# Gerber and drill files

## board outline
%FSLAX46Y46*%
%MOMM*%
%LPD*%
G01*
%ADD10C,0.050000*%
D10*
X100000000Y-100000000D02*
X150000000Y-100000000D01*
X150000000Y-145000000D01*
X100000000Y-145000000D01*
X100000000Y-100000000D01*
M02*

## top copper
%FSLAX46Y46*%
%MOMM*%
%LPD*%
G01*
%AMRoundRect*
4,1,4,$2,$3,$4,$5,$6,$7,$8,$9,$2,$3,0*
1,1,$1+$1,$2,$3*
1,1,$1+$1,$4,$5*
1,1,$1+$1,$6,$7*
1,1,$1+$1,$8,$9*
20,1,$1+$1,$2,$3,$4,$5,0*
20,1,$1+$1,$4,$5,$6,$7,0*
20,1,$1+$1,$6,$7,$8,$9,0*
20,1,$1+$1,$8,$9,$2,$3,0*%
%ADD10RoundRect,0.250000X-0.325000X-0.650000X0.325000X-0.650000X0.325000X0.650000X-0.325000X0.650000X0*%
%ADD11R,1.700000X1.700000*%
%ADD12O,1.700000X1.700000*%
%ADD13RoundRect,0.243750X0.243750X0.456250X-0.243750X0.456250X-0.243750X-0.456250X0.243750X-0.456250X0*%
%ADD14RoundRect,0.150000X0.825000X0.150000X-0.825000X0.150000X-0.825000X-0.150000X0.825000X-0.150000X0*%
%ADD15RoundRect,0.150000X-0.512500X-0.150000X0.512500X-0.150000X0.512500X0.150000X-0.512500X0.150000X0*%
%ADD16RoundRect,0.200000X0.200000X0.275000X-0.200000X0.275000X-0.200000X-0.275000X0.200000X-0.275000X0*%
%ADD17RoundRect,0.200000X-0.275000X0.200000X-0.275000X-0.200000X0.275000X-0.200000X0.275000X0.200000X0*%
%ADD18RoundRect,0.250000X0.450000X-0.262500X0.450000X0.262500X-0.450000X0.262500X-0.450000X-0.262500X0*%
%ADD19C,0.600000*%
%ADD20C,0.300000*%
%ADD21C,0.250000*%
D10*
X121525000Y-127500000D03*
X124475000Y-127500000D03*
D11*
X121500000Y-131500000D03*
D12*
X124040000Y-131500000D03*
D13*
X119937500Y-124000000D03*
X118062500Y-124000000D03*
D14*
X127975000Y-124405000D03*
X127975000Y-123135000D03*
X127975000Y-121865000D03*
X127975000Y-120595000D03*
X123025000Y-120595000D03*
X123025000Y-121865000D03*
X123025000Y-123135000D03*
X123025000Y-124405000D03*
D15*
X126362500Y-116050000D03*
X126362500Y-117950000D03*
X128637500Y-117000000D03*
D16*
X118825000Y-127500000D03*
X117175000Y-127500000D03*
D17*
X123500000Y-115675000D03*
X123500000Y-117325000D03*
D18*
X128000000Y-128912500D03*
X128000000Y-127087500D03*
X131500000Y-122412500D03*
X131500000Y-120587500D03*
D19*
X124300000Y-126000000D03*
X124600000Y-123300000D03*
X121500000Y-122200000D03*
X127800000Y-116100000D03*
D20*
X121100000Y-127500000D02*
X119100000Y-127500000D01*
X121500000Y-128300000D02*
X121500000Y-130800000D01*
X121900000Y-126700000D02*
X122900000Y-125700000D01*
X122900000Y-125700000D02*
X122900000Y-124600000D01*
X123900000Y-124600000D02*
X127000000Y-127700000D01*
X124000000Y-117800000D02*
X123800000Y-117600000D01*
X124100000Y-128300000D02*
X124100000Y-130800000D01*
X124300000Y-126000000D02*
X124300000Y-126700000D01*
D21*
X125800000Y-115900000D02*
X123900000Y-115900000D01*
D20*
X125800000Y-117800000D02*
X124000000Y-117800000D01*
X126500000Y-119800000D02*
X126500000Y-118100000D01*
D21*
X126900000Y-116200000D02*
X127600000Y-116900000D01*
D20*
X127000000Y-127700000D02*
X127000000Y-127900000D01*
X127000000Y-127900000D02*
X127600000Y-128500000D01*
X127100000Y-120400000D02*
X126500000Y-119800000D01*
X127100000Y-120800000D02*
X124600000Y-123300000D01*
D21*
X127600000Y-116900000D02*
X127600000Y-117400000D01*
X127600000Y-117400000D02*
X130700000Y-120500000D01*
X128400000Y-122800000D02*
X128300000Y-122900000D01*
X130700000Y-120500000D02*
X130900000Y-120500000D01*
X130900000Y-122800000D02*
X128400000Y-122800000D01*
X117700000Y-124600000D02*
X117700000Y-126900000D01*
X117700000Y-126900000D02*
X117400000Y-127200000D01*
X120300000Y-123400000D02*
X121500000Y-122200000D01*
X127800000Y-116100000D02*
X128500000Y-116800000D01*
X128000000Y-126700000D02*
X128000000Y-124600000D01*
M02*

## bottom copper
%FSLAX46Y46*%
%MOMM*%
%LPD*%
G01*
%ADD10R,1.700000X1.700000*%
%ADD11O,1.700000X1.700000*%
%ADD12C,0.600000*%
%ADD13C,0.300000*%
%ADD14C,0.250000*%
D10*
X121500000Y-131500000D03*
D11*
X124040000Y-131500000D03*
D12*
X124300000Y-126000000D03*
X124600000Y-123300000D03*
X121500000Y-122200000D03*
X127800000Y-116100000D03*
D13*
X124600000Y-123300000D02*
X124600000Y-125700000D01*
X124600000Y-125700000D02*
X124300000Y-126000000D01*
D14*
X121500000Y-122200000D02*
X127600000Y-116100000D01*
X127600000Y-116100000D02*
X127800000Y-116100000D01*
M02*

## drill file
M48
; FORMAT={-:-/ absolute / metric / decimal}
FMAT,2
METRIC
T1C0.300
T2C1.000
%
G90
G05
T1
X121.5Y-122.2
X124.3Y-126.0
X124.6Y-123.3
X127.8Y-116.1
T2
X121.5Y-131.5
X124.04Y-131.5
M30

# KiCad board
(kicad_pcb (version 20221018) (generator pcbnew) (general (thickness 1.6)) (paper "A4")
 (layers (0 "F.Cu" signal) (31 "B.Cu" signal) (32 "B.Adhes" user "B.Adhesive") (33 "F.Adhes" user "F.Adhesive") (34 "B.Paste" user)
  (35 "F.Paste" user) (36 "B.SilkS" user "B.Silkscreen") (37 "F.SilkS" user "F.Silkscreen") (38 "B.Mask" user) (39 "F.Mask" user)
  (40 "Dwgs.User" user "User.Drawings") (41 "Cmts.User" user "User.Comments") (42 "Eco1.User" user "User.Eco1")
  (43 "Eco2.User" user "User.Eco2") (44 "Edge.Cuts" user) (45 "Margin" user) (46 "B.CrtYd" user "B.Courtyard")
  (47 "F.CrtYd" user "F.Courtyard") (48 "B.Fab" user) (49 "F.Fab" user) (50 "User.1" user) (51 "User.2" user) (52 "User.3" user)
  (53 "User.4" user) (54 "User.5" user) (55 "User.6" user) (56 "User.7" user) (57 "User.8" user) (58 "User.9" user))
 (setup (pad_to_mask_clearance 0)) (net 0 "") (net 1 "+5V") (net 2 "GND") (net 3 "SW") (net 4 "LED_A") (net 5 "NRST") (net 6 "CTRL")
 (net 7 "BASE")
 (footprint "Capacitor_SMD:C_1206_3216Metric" (layer "F.Cu") (at 123 127.5)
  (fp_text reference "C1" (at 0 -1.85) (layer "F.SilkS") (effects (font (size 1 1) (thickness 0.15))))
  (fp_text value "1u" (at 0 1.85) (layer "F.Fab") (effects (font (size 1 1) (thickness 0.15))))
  (pad "1" smd roundrect (at -1.475 0) (size 1.15 1.8) (layers "F.Cu" "F.Paste" "F.Mask") (roundrect_rratio 0.217391) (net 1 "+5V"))
  (pad "2" smd roundrect (at 1.475 0) (size 1.15 1.8) (layers "F.Cu" "F.Paste" "F.Mask") (roundrect_rratio 0.217391) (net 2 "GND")))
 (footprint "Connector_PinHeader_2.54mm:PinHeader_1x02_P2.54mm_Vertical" (layer "F.Cu") (at 121.5 131.5 90)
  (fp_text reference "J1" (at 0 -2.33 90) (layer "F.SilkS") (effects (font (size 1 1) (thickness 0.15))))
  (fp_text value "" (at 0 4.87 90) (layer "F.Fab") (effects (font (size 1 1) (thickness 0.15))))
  (pad "1" thru_hole rect (at 0 0 90) (size 1.7 1.7) (drill 1) (layers "*.Cu" "*.Mask") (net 1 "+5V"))
  (pad "2" thru_hole oval (at 0 2.54 90) (size 1.7 1.7) (drill 1) (layers "*.Cu" "*.Mask") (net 2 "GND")))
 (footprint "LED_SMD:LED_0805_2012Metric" (layer "F.Cu") (at 119 124 180)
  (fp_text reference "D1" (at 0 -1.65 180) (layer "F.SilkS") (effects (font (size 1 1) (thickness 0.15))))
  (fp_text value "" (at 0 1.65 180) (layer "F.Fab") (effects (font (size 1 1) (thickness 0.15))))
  (pad "1" smd roundrect (at -0.9375 0 180) (size 0.975 1.4) (layers "F.Cu" "F.Paste" "F.Mask") (roundrect_rratio 0.25) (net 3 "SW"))
  (pad "2" smd roundrect (at 0.9375 0 180) (size 0.975 1.4) (layers "F.Cu" "F.Paste" "F.Mask") (roundrect_rratio 0.25) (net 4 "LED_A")))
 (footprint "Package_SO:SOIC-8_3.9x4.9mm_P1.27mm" (layer "F.Cu") (at 125.5 122.5 180)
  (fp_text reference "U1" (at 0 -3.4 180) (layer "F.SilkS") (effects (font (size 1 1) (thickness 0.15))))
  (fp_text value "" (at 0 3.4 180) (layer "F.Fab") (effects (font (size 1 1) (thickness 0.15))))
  (pad "1" smd roundrect (at -2.475 -1.905 180) (size 1.95 0.6) (layers "F.Cu" "F.Paste" "F.Mask") (roundrect_rratio 0.25) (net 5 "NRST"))
  (pad "2" smd roundrect (at -2.475 -0.635 180) (size 1.95 0.6) (layers "F.Cu" "F.Paste" "F.Mask") (roundrect_rratio 0.25) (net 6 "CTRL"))
  (pad "3" smd roundrect (at -2.475 0.635 180) (size 1.95 0.6) (layers "F.Cu" "F.Paste" "F.Mask") (roundrect_rratio 0.25))
  (pad "4" smd roundrect (at -2.475 1.905 180) (size 1.95 0.6) (layers "F.Cu" "F.Paste" "F.Mask") (roundrect_rratio 0.25) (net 2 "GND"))
  (pad "5" smd roundrect (at 2.475 1.905 180) (size 1.95 0.6) (layers "F.Cu" "F.Paste" "F.Mask") (roundrect_rratio 0.25))
  (pad "6" smd roundrect (at 2.475 0.635 180) (size 1.95 0.6) (layers "F.Cu" "F.Paste" "F.Mask") (roundrect_rratio 0.25))
  (pad "7" smd roundrect (at 2.475 -0.635 180) (size 1.95 0.6) (layers "F.Cu" "F.Paste" "F.Mask") (roundrect_rratio 0.25))
  (pad "8" smd roundrect (at 2.475 -1.905 180) (size 1.95 0.6) (layers "F.Cu" "F.Paste" "F.Mask") (roundrect_rratio 0.25) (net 1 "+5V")))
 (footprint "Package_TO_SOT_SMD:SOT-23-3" (layer "F.Cu") (at 127.5 117)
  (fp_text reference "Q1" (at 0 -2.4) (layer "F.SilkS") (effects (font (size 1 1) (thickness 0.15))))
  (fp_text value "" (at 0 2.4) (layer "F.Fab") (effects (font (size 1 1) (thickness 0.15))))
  (pad "1" smd roundrect (at -1.1375 -0.95) (size 1.325 0.6) (layers "F.Cu" "F.Paste" "F.Mask") (roundrect_rratio 0.25) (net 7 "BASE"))
  (pad "2" smd roundrect (at -1.1375 0.95) (size 1.325 0.6) (layers "F.Cu" "F.Paste" "F.Mask") (roundrect_rratio 0.25) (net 2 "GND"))
  (pad "3" smd roundrect (at 1.1375 0) (size 1.325 0.6) (layers "F.Cu" "F.Paste" "F.Mask") (roundrect_rratio 0.25) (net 3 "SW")))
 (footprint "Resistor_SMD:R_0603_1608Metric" (layer "F.Cu") (at 118 127.5 180)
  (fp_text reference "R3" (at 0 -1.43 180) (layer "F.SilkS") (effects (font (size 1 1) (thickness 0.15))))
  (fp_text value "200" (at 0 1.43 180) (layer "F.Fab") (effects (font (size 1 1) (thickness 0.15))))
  (pad "1" smd roundrect (at -0.825 0 180) (size 0.8 0.95) (layers "F.Cu" "F.Paste" "F.Mask") (roundrect_rratio 0.25) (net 1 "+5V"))
  (pad "2" smd roundrect (at 0.825 0 180) (size 0.8 0.95) (layers "F.Cu" "F.Paste" "F.Mask") (roundrect_rratio 0.25) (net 4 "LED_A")))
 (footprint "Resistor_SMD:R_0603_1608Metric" (layer "F.Cu") (at 123.5 116.5 -90)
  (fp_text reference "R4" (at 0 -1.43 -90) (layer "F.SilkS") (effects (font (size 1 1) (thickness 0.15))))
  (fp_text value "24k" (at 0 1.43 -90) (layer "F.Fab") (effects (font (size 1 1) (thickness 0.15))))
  (pad "1" smd roundrect (at -0.825 0 270) (size 0.8 0.95) (layers "F.Cu" "F.Paste" "F.Mask") (roundrect_rratio 0.25) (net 7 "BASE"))
  (pad "2" smd roundrect (at 0.825 0 270) (size 0.8 0.95) (layers "F.Cu" "F.Paste" "F.Mask") (roundrect_rratio 0.25) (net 2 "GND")))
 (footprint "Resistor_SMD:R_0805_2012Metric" (layer "F.Cu") (at 128 128 90)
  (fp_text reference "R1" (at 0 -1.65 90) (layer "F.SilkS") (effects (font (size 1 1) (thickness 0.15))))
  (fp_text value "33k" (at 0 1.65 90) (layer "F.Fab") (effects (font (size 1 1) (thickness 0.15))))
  (pad "1" smd roundrect (at -0.9125 0 90) (size 1.025 1.4) (layers "F.Cu" "F.Paste" "F.Mask") (roundrect_rratio 0.243902) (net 1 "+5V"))
  (pad "2" smd roundrect (at 0.9125 0 90) (size 1.025 1.4) (layers "F.Cu" "F.Paste" "F.Mask") (roundrect_rratio 0.243902) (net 5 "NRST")))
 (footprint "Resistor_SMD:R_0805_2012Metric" (layer "F.Cu") (at 131.5 121.5 90)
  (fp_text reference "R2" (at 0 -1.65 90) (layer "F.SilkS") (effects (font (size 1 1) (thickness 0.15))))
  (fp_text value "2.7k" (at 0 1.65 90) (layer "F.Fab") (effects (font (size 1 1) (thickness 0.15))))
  (pad "1" smd roundrect (at -0.9125 0 90) (size 1.025 1.4) (layers "F.Cu" "F.Paste" "F.Mask") (roundrect_rratio 0.243902) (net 6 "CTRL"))
  (pad "2" smd roundrect (at 0.9125 0 90) (size 1.025 1.4) (layers "F.Cu" "F.Paste" "F.Mask") (roundrect_rratio 0.243902) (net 7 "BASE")))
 (gr_rect (start 100 100) (end 150 145) (stroke (width 0.05) (type default)) (fill none) (layer "Edge.Cuts"))
 (segment (start 121.1 127.5) (end 119.1 127.5) (width 0.3) (layer "F.Cu") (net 1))
 (segment (start 121.5 128.3) (end 121.5 130.8) (width 0.3) (layer "F.Cu") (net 1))
 (segment (start 121.9 126.7) (end 122.9 125.7) (width 0.3) (layer "F.Cu") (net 1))
 (segment (start 122.9 125.7) (end 122.9 124.6) (width 0.3) (layer "F.Cu") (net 1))
 (segment (start 123.9 124.6) (end 127 127.7) (width 0.3) (layer "F.Cu") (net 1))
 (segment (start 124 117.8) (end 123.8 117.6) (width 0.3) (layer "F.Cu") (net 2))
 (segment (start 124.1 128.3) (end 124.1 130.8) (width 0.3) (layer "F.Cu") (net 2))
 (segment (start 124.3 126) (end 124.3 126.7) (width 0.3) (layer "F.Cu") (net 2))
 (segment (start 125.8 115.9) (end 123.9 115.9) (width 0.25) (layer "F.Cu") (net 7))
 (segment (start 125.8 117.8) (end 124 117.8) (width 0.3) (layer "F.Cu") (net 2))
 (segment (start 126.5 119.8) (end 126.5 118.1) (width 0.3) (layer "F.Cu") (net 2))
 (segment (start 126.9 116.2) (end 127.6 116.9) (width 0.25) (layer "F.Cu") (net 7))
 (segment (start 127 127.7) (end 127 127.9) (width 0.3) (layer "F.Cu") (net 1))
 (segment (start 127 127.9) (end 127.6 128.5) (width 0.3) (layer "F.Cu") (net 1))
 (segment (start 127.1 120.4) (end 126.5 119.8) (width 0.3) (layer "F.Cu") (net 2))
 (segment (start 127.1 120.8) (end 124.6 123.3) (width 0.3) (layer "F.Cu") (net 2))
 (segment (start 127.6 116.9) (end 127.6 117.4) (width 0.25) (layer "F.Cu") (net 7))
 (segment (start 127.6 117.4) (end 130.7 120.5) (width 0.25) (layer "F.Cu") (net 7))
 (segment (start 128.4 122.8) (end 128.3 122.9) (width 0.25) (layer "F.Cu") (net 6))
 (segment (start 130.7 120.5) (end 130.9 120.5) (width 0.25) (layer "F.Cu") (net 7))
 (segment (start 130.9 122.8) (end 128.4 122.8) (width 0.25) (layer "F.Cu") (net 6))
 (via (at 124.3 126) (size 0.6) (drill 0.3) (layers "F.Cu" "B.Cu") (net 2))
 (via (at 124.6 123.3) (size 0.6) (drill 0.3) (layers "F.Cu" "B.Cu") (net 2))
 (segment (start 117.7 124.6) (end 117.7 126.9) (width 0.25) (layer "F.Cu") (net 4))
 (segment (start 117.7 126.9) (end 117.4 127.2) (width 0.25) (layer "F.Cu") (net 4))
 (segment (start 120.3 123.4) (end 121.5 122.2) (width 0.25) (layer "F.Cu") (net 3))
 (segment (start 124.6 123.3) (end 124.6 125.7) (width 0.3) (layer "B.Cu") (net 2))
 (segment (start 124.6 125.7) (end 124.3 126) (width 0.3) (layer "B.Cu") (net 2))
 (segment (start 127.8 116.1) (end 128.5 116.8) (width 0.25) (layer "F.Cu") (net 3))
 (segment (start 128 126.7) (end 128 124.6) (width 0.25) (layer "F.Cu") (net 5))
 (via (at 121.5 122.2) (size 0.6) (drill 0.3) (layers "F.Cu" "B.Cu") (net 3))
 (via (at 127.8 116.1) (size 0.6) (drill 0.3) (layers "F.Cu" "B.Cu") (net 3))
 (segment (start 121.5 122.2) (end 127.6 116.1) (width 0.25) (layer "B.Cu") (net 3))
 (segment (start 127.6 116.1) (end 127.8 116.1) (width 0.25) (layer "B.Cu") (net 3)))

